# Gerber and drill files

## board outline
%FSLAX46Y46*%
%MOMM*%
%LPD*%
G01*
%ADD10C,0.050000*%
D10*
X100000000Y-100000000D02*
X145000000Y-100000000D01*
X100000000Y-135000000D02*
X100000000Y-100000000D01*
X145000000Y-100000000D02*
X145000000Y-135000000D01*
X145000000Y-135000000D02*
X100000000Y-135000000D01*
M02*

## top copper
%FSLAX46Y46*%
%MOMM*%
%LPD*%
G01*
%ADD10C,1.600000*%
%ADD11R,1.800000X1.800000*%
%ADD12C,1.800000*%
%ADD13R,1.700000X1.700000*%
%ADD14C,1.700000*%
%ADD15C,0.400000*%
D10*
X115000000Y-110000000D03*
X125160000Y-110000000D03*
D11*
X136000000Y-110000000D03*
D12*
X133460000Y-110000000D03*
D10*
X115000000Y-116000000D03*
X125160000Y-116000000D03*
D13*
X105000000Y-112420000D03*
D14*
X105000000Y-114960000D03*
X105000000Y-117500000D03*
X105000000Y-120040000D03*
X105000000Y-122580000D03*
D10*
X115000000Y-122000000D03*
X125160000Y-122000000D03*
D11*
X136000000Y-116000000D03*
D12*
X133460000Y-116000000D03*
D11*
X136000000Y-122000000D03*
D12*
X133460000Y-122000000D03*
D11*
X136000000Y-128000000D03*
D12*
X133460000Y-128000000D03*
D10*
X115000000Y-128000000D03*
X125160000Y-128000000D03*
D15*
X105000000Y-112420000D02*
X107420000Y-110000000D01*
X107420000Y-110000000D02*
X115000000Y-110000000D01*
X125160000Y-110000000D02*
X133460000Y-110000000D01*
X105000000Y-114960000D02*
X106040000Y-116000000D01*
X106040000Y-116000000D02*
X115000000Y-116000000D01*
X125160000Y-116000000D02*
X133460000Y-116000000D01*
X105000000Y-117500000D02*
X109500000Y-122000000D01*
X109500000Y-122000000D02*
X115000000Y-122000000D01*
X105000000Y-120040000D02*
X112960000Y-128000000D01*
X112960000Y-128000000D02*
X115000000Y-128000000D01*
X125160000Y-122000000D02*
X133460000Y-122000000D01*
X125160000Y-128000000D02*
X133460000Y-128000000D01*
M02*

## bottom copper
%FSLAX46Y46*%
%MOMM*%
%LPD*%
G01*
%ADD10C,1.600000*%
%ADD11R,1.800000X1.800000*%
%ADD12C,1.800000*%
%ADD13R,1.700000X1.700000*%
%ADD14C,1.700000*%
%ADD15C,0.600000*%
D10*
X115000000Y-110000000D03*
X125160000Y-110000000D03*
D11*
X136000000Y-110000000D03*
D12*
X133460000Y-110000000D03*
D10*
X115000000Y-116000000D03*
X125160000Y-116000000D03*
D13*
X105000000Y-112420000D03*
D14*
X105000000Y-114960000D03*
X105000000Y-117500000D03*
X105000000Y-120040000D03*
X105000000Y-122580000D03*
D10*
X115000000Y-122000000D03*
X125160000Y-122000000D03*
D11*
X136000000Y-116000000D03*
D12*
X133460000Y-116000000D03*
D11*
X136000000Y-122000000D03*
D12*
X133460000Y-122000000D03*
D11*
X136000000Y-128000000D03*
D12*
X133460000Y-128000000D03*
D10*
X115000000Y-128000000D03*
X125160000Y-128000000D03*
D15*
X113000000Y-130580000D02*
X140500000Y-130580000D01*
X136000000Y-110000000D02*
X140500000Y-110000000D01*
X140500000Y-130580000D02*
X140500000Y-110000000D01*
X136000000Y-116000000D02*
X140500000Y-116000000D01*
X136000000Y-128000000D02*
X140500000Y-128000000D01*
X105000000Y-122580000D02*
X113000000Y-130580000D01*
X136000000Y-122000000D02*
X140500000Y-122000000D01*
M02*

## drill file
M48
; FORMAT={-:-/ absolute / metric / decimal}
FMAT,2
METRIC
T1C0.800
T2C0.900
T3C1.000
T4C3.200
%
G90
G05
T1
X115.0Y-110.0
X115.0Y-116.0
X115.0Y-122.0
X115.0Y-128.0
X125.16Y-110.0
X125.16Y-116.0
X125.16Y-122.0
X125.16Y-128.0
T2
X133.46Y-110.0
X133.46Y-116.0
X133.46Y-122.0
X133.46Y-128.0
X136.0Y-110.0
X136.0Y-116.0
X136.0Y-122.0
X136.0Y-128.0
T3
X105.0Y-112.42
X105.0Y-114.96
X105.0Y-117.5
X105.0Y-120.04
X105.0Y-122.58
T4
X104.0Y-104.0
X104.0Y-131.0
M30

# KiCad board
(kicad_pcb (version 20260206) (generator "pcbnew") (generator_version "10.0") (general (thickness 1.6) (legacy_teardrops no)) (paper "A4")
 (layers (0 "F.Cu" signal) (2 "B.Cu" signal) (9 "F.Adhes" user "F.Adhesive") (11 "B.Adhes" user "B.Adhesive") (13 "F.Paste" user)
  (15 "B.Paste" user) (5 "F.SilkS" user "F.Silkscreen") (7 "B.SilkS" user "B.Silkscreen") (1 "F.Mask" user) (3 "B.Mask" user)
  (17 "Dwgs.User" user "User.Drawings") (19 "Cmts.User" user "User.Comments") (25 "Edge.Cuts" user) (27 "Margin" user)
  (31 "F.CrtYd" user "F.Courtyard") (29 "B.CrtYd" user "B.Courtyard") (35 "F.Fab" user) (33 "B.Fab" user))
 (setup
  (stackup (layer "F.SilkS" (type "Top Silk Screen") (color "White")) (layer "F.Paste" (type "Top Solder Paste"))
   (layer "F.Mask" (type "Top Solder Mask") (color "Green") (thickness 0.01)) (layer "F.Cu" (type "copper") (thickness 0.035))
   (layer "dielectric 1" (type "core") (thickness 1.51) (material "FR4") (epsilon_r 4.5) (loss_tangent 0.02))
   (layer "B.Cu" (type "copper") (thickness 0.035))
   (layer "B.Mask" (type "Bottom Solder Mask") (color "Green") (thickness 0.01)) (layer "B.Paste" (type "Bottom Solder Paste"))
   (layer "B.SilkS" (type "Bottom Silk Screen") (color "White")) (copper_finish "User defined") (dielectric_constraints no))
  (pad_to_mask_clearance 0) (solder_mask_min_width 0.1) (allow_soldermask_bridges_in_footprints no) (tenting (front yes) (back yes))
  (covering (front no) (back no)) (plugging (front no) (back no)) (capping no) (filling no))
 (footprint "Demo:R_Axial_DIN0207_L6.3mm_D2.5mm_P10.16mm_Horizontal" (layer "F.Cu") (at 115 110)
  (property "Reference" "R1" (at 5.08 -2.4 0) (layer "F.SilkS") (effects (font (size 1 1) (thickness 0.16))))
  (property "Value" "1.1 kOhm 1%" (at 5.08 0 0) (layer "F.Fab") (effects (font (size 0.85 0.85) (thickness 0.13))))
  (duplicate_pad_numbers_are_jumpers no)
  (pad "1" thru_hole circle (at 0 0) (size 1.6 1.6) (drill 0.8) (layers "*.Cu" "*.Mask") (remove_unused_layers no) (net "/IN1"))
  (pad "2" thru_hole circle (at 10.16 0) (size 1.6 1.6) (drill 0.8) (layers "*.Cu" "*.Mask") (remove_unused_layers no) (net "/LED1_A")))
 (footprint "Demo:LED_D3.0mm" (layer "F.Cu") (at 136 110 180)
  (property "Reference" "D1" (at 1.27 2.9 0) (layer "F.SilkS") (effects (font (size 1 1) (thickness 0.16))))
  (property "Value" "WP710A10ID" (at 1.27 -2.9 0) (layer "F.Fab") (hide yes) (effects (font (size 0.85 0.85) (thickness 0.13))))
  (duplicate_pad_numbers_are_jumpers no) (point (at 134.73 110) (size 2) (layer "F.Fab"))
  (pad "1" thru_hole rect (at 0 0 180) (size 1.8 1.8) (drill 0.9) (layers "*.Cu" "*.Mask") (remove_unused_layers no) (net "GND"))
  (pad "2" thru_hole circle (at 2.54 0 180) (size 1.8 1.8) (drill 0.9) (layers "*.Cu" "*.Mask") (remove_unused_layers no) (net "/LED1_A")))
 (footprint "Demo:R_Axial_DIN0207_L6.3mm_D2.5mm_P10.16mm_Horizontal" (layer "F.Cu") (at 115 116)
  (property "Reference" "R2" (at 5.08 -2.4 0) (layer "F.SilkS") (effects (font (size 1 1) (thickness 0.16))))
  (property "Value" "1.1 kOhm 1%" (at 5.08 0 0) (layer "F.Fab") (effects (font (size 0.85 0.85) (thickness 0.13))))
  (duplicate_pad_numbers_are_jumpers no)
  (pad "1" thru_hole circle (at 0 0) (size 1.6 1.6) (drill 0.8) (layers "*.Cu" "*.Mask") (remove_unused_layers no) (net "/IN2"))
  (pad "2" thru_hole circle (at 10.16 0) (size 1.6 1.6) (drill 0.8) (layers "*.Cu" "*.Mask") (remove_unused_layers no) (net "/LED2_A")))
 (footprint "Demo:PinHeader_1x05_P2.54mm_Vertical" (layer "F.Cu") (at 105 112.42)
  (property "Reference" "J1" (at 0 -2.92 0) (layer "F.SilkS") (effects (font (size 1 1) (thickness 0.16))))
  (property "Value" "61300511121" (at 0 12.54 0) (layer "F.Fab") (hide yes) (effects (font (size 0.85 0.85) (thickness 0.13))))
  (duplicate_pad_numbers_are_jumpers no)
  (pad "1" thru_hole rect (at 0 0) (size 1.7 1.7) (drill 1) (layers "*.Cu" "*.Mask") (remove_unused_layers no) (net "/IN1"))
  (pad "2" thru_hole circle (at 0 2.54) (size 1.7 1.7) (drill 1) (layers "*.Cu" "*.Mask") (remove_unused_layers no) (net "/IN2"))
  (pad "3" thru_hole circle (at 0 5.08) (size 1.7 1.7) (drill 1) (layers "*.Cu" "*.Mask") (remove_unused_layers no) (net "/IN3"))
  (pad "4" thru_hole circle (at 0 7.62) (size 1.7 1.7) (drill 1) (layers "*.Cu" "*.Mask") (remove_unused_layers no) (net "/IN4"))
  (pad "5" thru_hole circle (at 0 10.16) (size 1.7 1.7) (drill 1) (layers "*.Cu" "*.Mask") (remove_unused_layers no) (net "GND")))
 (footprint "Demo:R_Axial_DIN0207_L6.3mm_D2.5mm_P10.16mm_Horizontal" (layer "F.Cu") (at 115 122)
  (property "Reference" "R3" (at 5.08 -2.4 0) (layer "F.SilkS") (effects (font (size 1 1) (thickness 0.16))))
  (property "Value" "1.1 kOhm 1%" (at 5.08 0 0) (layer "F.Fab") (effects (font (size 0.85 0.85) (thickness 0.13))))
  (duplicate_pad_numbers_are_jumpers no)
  (pad "1" thru_hole circle (at 0 0) (size 1.6 1.6) (drill 0.8) (layers "*.Cu" "*.Mask") (remove_unused_layers no) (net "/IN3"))
  (pad "2" thru_hole circle (at 10.16 0) (size 1.6 1.6) (drill 0.8) (layers "*.Cu" "*.Mask") (remove_unused_layers no) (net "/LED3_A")))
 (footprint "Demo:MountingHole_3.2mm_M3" (layer "F.Cu") (at 104 104)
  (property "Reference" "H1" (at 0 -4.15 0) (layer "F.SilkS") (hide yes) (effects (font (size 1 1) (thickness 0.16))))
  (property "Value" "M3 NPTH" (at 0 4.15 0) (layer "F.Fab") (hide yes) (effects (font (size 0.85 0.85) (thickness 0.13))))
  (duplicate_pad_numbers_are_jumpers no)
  (pad "" np_thru_hole circle (at 0 0) (size 3.2 3.2) (drill 3.2) (layers "*.Cu" "*.Mask")))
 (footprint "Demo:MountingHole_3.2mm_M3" (layer "F.Cu") (at 104 131)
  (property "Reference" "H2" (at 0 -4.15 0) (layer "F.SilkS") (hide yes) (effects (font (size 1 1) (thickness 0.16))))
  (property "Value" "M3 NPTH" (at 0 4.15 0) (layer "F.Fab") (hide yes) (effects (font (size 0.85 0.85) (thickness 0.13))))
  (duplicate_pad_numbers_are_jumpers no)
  (pad "" np_thru_hole circle (at 0 0) (size 3.2 3.2) (drill 3.2) (layers "*.Cu" "*.Mask")))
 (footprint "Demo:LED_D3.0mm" (layer "F.Cu") (at 136 116 180)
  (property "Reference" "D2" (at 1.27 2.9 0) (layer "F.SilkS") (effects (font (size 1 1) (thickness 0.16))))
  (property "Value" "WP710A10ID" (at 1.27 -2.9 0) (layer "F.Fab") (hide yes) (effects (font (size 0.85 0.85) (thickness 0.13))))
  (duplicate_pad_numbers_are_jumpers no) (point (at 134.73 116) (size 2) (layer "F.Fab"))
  (pad "1" thru_hole rect (at 0 0 180) (size 1.8 1.8) (drill 0.9) (layers "*.Cu" "*.Mask") (remove_unused_layers no) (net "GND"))
  (pad "2" thru_hole circle (at 2.54 0 180) (size 1.8 1.8) (drill 0.9) (layers "*.Cu" "*.Mask") (remove_unused_layers no) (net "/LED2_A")))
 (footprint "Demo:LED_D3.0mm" (layer "F.Cu") (at 136 122 180)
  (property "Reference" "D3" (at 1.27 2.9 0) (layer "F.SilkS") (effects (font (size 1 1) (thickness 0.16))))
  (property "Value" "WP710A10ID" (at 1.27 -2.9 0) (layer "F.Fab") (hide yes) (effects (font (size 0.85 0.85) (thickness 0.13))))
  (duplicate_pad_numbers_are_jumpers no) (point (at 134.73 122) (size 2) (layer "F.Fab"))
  (pad "1" thru_hole rect (at 0 0 180) (size 1.8 1.8) (drill 0.9) (layers "*.Cu" "*.Mask") (remove_unused_layers no) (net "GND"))
  (pad "2" thru_hole circle (at 2.54 0 180) (size 1.8 1.8) (drill 0.9) (layers "*.Cu" "*.Mask") (remove_unused_layers no) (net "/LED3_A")))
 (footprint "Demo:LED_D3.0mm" (layer "F.Cu") (at 136 128 180)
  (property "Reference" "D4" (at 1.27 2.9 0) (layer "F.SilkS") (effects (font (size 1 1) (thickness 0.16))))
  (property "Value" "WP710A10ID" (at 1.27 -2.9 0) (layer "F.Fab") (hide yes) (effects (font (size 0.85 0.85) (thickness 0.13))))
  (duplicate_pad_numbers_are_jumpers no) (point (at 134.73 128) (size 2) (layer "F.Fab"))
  (pad "1" thru_hole rect (at 0 0 180) (size 1.8 1.8) (drill 0.9) (layers "*.Cu" "*.Mask") (remove_unused_layers no) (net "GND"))
  (pad "2" thru_hole circle (at 2.54 0 180) (size 1.8 1.8) (drill 0.9) (layers "*.Cu" "*.Mask") (remove_unused_layers no) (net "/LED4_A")))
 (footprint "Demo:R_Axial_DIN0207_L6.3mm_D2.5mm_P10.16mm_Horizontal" (layer "F.Cu") (at 115 128)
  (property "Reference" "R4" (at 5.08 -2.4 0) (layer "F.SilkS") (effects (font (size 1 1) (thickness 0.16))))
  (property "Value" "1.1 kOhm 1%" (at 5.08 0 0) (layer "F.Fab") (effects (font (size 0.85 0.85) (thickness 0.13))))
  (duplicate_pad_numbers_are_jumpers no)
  (pad "1" thru_hole circle (at 0 0) (size 1.6 1.6) (drill 0.8) (layers "*.Cu" "*.Mask") (remove_unused_layers no) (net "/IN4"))
  (pad "2" thru_hole circle (at 10.16 0) (size 1.6 1.6) (drill 0.8) (layers "*.Cu" "*.Mask") (remove_unused_layers no) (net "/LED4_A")))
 (gr_line (start 100 100) (end 145 100) (stroke (width 0.05) (type default)) (layer "Edge.Cuts"))
 (gr_line (start 100 135) (end 100 100) (stroke (width 0.05) (type default)) (layer "Edge.Cuts"))
 (gr_line (start 145 100) (end 145 135) (stroke (width 0.05) (type default)) (layer "Edge.Cuts"))
 (gr_line (start 145 135) (end 100 135) (stroke (width 0.05) (type default)) (layer "Edge.Cuts"))
 (segment (start 105 112.42) (end 107.42 110) (width 0.4) (layer "F.Cu") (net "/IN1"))
 (segment (start 107.42 110) (end 115 110) (width 0.4) (layer "F.Cu") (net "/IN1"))
 (segment (start 125.16 110) (end 133.46 110) (width 0.4) (layer "F.Cu") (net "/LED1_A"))
 (segment (start 113 130.58) (end 140.5 130.58) (width 0.6) (layer "B.Cu") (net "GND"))
 (segment (start 136 110) (end 140.5 110) (width 0.6) (layer "B.Cu") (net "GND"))
 (segment (start 140.5 130.58) (end 140.5 110) (width 0.6) (layer "B.Cu") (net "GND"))
 (segment (start 136 116) (end 140.5 116) (width 0.6) (layer "B.Cu") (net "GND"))
 (segment (start 136 128) (end 140.5 128) (width 0.6) (layer "B.Cu") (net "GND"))
 (segment (start 105 122.58) (end 113 130.58) (width 0.6) (layer "B.Cu") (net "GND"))
 (segment (start 136 122) (end 140.5 122) (width 0.6) (layer "B.Cu") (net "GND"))
 (segment (start 105 114.96) (end 106.04 116) (width 0.4) (layer "F.Cu") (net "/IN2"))
 (segment (start 106.04 116) (end 115 116) (width 0.4) (layer "F.Cu") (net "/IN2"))
 (segment (start 125.16 116) (end 133.46 116) (width 0.4) (layer "F.Cu") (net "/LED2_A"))
 (segment (start 105 117.5) (end 109.5 122) (width 0.4) (layer "F.Cu") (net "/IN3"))
 (segment (start 109.5 122) (end 115 122) (width 0.4) (layer "F.Cu") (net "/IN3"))
 (segment (start 105 120.04) (end 112.96 128) (width 0.4) (layer "F.Cu") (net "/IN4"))
 (segment (start 112.96 128) (end 115 128) (width 0.4) (layer "F.Cu") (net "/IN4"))
 (segment (start 125.16 122) (end 133.46 122) (width 0.4) (layer "F.Cu") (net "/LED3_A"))
 (segment (start 125.16 128) (end 133.46 128) (width 0.4) (layer "F.Cu") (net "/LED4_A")))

